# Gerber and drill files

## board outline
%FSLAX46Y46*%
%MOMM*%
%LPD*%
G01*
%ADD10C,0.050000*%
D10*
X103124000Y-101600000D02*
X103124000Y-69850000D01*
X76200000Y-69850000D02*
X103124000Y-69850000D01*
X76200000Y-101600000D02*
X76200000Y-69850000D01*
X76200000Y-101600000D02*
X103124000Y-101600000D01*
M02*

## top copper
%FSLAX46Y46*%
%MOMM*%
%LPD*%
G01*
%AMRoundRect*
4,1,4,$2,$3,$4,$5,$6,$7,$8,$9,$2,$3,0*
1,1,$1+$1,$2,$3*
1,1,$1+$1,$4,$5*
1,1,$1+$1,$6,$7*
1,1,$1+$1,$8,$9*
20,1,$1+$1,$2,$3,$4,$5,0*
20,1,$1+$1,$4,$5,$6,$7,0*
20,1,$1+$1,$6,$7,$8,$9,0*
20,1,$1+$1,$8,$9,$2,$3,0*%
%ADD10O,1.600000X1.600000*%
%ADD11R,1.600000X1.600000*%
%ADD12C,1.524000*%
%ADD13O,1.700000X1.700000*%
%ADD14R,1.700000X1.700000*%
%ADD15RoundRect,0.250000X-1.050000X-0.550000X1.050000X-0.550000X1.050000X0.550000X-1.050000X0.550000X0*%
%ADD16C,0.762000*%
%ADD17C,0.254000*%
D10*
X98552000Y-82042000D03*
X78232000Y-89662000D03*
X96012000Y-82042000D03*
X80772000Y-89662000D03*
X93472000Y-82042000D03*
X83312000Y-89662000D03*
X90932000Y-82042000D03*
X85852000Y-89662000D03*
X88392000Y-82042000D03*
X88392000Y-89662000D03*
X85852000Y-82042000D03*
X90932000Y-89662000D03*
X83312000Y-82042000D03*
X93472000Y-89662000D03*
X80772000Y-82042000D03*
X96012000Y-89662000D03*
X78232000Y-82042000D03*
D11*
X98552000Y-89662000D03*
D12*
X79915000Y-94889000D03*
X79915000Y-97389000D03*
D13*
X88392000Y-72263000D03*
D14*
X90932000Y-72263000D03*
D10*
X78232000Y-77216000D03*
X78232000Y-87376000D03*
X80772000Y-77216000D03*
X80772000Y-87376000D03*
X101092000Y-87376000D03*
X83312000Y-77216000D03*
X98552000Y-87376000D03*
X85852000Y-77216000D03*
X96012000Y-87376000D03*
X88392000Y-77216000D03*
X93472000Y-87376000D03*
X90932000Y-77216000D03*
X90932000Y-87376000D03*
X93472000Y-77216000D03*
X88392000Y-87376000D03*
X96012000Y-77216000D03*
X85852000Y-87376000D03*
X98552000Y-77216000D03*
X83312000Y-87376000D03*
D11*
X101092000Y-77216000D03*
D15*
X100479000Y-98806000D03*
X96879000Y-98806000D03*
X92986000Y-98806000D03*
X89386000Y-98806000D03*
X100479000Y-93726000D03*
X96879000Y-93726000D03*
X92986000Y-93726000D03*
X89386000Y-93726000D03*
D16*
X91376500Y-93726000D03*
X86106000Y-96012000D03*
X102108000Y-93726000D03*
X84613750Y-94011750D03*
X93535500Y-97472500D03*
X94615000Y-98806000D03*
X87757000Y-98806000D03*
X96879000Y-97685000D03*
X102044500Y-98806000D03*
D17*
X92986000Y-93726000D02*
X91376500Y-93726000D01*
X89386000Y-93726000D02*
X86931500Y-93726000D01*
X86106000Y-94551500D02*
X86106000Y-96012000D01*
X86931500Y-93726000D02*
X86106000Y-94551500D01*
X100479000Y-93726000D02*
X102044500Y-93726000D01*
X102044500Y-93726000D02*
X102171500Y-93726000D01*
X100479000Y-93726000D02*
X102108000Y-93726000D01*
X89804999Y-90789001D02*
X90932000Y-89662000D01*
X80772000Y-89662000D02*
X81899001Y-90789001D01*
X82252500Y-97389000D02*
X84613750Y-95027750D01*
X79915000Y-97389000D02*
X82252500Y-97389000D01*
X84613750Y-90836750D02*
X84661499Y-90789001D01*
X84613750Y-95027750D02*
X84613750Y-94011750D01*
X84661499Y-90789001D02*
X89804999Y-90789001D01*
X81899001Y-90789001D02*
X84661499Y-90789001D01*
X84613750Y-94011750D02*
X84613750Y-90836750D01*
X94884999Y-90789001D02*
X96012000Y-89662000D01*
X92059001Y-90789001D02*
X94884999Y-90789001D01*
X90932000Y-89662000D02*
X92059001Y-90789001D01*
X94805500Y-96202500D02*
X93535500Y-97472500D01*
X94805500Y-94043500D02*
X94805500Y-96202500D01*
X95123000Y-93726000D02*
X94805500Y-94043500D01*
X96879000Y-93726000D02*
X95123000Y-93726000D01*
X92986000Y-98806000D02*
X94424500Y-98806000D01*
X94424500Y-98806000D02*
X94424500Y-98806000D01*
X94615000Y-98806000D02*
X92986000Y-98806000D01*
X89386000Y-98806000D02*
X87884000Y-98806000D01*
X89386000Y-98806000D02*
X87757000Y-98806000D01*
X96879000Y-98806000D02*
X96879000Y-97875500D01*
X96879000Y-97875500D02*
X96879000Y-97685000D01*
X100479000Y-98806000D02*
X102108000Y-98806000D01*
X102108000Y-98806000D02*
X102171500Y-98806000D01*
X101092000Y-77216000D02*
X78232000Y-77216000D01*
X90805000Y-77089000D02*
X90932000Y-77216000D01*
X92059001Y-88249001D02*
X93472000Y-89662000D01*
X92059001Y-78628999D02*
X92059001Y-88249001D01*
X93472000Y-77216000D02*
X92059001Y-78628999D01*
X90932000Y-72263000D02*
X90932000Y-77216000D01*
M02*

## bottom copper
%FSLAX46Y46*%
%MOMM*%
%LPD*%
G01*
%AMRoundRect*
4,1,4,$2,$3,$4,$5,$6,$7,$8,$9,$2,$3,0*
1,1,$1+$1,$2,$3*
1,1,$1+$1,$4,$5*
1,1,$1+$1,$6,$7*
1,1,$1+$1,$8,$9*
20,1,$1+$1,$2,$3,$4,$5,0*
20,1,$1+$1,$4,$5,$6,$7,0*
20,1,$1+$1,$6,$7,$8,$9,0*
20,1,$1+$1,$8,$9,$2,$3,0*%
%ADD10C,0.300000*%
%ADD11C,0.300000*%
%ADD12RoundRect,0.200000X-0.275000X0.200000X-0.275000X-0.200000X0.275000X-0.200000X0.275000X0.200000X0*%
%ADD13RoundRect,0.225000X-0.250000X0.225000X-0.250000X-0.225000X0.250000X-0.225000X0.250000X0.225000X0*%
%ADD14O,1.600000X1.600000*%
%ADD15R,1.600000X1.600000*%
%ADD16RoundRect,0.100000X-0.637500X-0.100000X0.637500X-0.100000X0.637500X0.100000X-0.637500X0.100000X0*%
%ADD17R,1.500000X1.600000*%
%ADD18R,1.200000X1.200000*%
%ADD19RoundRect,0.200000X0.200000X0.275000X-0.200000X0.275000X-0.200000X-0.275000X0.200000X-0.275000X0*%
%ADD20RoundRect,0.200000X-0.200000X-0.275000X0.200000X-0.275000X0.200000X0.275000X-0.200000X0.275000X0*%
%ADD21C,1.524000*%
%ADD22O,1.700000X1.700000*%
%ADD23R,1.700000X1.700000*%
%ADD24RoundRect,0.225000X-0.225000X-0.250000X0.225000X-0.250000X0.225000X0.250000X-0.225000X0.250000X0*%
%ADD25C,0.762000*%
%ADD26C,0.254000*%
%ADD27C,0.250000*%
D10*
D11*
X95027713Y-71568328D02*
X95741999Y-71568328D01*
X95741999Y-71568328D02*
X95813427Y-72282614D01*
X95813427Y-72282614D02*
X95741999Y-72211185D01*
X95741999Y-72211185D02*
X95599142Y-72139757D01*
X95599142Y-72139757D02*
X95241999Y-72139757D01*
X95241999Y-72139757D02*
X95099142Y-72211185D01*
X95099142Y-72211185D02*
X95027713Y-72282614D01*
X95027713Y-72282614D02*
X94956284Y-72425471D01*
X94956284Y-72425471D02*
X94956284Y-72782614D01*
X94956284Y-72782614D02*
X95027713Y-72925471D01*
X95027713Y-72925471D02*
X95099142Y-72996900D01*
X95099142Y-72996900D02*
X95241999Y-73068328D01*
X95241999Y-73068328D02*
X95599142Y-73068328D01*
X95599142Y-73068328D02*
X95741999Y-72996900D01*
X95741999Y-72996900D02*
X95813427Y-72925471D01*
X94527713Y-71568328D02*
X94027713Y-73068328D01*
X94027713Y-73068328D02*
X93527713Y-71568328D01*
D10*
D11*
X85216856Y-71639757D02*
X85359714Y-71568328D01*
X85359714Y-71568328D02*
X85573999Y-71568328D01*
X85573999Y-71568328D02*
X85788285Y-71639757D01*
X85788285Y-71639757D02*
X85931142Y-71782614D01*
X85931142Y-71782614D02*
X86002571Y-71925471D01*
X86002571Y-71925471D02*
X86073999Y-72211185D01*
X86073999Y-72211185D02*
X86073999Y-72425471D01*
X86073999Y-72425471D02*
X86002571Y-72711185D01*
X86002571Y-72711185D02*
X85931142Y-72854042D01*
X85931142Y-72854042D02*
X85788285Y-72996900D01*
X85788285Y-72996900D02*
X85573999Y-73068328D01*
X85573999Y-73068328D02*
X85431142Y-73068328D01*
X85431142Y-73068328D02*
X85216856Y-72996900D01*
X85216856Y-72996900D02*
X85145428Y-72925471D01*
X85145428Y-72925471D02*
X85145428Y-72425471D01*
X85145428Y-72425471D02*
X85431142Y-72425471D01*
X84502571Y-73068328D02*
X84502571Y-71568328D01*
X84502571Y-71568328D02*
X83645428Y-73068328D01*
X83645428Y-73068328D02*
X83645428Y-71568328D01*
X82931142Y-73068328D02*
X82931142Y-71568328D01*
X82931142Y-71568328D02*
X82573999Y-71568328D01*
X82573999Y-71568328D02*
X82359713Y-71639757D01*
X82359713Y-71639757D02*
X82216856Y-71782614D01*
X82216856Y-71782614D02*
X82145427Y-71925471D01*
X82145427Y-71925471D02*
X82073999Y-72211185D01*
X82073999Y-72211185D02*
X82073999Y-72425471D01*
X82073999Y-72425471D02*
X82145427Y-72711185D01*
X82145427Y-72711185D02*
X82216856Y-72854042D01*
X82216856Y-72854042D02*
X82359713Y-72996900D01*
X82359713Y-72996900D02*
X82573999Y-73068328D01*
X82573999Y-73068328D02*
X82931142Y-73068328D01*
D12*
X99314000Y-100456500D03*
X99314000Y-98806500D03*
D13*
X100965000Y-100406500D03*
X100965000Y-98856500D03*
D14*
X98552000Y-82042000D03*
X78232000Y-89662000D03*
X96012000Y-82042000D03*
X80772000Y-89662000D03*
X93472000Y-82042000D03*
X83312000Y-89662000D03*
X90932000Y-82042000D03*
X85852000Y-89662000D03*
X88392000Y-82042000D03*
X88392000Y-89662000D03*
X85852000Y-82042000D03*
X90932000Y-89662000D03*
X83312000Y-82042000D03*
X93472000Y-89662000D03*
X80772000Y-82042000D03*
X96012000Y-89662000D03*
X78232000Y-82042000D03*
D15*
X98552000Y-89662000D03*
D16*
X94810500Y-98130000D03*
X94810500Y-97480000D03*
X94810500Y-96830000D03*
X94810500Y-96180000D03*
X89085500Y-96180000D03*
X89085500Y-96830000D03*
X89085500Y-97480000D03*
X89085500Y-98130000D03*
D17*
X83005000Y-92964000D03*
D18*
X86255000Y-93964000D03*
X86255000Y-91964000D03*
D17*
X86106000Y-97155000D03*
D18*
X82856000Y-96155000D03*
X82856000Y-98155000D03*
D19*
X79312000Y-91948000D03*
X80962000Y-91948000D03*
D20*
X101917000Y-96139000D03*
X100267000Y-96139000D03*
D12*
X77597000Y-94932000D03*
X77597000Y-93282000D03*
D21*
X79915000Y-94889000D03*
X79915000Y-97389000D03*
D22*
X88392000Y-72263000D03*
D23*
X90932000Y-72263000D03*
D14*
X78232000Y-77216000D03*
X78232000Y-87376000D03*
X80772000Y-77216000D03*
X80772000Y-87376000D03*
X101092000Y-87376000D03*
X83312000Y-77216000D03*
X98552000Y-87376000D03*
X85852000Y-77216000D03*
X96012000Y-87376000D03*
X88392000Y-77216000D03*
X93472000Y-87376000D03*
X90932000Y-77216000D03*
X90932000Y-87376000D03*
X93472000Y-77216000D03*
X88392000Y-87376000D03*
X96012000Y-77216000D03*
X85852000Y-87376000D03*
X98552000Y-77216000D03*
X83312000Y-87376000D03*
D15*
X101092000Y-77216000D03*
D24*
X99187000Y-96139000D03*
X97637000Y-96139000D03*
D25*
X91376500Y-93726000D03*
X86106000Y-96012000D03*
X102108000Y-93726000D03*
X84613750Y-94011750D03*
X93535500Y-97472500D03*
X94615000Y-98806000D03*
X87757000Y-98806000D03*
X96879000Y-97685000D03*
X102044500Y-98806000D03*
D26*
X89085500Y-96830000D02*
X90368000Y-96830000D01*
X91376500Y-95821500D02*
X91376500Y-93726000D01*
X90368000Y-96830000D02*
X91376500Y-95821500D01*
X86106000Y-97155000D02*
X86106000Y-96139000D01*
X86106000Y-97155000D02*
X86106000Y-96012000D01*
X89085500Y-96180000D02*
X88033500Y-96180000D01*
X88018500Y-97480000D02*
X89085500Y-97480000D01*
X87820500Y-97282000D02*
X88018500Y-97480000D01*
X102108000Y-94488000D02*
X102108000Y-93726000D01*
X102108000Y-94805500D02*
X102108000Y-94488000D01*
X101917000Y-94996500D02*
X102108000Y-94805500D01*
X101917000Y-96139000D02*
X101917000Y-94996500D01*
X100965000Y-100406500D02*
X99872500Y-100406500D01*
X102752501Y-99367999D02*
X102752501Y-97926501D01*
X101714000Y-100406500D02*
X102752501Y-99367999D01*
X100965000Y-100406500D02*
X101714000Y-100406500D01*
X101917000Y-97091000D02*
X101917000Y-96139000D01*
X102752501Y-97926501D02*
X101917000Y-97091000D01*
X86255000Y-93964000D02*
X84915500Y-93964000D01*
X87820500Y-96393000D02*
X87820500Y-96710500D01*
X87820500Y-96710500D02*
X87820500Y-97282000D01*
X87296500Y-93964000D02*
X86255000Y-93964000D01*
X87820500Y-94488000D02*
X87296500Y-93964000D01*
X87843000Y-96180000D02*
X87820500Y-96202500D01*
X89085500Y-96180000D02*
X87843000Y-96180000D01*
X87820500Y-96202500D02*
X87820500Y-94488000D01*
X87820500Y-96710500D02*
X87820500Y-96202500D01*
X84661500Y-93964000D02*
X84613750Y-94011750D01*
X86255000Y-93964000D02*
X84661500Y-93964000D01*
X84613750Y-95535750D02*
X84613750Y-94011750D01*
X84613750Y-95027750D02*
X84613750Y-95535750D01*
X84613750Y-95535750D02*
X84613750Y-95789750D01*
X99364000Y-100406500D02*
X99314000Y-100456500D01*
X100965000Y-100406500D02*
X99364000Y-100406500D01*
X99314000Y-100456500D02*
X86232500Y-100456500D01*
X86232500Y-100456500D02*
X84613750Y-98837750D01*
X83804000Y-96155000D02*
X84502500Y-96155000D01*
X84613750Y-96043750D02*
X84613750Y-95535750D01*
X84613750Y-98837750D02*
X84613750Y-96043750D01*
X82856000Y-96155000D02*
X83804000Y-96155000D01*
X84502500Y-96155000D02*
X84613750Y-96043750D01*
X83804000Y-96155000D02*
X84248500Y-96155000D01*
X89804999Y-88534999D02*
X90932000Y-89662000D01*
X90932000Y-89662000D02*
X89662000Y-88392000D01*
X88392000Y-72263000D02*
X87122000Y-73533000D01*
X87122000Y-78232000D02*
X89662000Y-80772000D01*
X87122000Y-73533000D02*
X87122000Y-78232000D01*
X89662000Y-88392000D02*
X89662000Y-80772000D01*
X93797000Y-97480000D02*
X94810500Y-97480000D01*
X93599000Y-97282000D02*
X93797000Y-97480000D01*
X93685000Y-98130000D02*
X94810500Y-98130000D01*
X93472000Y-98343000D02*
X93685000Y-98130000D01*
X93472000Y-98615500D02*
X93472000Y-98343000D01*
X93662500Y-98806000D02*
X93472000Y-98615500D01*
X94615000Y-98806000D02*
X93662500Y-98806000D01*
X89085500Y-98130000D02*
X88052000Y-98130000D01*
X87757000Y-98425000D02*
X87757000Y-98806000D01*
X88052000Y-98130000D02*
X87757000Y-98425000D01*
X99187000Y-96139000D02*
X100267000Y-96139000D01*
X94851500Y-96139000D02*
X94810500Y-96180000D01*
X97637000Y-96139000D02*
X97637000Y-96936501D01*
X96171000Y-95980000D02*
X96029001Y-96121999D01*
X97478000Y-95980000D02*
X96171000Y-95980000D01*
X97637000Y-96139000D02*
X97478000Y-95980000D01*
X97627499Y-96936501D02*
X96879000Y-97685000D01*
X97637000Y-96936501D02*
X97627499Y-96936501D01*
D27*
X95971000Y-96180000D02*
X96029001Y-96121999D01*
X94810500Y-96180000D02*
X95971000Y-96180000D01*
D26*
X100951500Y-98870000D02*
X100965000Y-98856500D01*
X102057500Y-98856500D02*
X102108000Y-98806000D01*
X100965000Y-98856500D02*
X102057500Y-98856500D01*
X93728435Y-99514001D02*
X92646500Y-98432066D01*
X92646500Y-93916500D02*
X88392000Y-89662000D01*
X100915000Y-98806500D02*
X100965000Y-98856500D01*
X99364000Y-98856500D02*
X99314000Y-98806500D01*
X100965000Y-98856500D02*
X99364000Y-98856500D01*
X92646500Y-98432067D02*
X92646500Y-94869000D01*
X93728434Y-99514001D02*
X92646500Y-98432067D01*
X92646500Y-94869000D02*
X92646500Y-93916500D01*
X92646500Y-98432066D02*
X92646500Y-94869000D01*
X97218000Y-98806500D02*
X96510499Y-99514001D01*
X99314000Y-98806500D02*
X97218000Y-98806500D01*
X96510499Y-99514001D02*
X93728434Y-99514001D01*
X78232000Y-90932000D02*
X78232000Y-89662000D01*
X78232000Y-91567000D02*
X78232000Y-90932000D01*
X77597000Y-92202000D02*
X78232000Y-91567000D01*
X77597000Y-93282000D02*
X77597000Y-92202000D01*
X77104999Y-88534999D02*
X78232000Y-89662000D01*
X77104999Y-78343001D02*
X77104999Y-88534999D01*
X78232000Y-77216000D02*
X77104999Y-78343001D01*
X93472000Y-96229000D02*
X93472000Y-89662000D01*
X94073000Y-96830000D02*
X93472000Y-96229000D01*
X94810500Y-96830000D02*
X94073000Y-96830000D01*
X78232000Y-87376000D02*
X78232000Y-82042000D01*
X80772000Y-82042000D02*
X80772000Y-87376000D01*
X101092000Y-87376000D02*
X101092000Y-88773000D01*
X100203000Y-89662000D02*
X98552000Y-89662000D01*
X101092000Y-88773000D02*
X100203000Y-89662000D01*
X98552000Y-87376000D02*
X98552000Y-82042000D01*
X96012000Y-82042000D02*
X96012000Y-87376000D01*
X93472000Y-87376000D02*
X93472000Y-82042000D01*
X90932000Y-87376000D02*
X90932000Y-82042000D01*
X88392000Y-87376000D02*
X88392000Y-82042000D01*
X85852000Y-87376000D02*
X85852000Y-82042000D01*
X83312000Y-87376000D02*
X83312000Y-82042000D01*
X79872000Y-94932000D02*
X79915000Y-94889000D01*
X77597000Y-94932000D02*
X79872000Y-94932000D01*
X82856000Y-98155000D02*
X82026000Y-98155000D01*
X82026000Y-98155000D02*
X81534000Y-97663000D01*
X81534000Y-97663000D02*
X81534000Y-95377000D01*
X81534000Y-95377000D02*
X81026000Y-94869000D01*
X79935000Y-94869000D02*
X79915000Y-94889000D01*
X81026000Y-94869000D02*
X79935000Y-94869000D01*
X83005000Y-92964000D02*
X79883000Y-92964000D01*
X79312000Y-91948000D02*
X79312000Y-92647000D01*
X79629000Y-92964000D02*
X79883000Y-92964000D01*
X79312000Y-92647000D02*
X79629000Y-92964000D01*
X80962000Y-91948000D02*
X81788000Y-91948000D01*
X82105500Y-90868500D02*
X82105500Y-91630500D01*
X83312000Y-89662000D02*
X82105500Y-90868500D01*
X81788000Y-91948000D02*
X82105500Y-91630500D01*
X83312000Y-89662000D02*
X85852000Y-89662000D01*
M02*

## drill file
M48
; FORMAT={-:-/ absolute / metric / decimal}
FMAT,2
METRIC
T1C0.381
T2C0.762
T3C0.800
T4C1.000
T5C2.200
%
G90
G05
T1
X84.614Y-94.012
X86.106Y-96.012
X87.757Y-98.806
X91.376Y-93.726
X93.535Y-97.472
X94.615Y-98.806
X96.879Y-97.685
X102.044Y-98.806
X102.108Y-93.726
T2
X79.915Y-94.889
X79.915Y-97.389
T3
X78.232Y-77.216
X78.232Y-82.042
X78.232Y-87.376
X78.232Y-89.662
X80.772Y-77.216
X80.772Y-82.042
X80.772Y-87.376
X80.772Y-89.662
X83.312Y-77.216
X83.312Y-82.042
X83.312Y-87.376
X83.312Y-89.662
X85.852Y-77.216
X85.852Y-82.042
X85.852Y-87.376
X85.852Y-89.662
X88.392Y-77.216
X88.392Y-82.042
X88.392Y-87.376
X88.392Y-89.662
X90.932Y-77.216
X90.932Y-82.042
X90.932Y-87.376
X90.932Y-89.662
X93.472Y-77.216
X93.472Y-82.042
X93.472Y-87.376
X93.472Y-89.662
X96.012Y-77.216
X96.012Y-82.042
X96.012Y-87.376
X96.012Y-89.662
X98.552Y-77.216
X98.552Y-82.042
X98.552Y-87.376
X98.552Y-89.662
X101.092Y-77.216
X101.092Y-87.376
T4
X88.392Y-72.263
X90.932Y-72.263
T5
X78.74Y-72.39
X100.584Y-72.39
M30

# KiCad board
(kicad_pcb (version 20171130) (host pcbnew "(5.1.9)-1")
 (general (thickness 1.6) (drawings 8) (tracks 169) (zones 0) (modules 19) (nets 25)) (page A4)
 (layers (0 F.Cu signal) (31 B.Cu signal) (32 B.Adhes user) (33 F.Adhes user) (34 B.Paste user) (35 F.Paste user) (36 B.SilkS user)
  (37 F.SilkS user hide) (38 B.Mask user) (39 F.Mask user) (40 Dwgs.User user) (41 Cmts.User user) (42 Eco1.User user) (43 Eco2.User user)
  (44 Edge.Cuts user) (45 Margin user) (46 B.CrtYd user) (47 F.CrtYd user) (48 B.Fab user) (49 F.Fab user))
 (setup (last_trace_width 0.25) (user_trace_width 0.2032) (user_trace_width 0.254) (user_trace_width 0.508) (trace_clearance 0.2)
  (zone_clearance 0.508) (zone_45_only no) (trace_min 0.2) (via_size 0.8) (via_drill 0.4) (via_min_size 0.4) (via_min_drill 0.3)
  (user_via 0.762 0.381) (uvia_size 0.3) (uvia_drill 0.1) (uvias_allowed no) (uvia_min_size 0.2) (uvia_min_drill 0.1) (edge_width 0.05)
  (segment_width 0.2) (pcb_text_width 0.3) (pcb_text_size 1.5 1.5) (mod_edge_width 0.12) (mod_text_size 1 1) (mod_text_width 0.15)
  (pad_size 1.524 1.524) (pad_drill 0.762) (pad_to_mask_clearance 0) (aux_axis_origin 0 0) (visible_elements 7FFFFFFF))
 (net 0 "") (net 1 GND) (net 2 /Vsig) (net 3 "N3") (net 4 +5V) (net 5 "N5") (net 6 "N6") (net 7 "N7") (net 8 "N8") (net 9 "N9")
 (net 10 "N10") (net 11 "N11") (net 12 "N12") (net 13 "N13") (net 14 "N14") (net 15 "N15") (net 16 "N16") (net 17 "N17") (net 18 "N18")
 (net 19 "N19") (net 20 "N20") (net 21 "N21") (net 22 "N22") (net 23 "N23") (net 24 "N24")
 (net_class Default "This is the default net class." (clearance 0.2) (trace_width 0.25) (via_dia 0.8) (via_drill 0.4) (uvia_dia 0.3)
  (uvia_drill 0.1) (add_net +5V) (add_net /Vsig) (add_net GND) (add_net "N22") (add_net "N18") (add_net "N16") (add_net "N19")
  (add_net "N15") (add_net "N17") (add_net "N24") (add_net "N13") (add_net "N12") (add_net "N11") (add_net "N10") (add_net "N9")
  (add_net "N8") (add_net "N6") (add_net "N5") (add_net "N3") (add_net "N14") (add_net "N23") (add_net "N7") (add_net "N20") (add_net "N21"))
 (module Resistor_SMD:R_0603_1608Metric (layer B.Cu) (at 99.314 99.6315 270)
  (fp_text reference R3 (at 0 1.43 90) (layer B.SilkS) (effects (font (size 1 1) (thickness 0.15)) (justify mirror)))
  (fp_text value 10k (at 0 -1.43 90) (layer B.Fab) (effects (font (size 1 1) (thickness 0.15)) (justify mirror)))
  (pad 2 smd roundrect (at 0.825 0 270) (size 0.8 0.95) (layers B.Cu B.Paste B.Mask) (roundrect_rratio 0.25) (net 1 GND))
  (pad 1 smd roundrect (at -0.825 0 270) (size 0.8 0.95) (layers B.Cu B.Paste B.Mask) (roundrect_rratio 0.25) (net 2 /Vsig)))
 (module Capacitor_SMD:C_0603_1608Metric (layer B.Cu) (at 100.965 99.6315 270)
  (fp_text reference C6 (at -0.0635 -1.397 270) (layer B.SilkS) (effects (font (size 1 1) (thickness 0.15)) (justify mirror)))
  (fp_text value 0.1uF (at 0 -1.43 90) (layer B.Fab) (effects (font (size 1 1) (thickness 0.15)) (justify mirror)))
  (pad 2 smd roundrect (at 0.775 0 270) (size 0.9 0.95) (layers B.Cu B.Paste B.Mask) (roundrect_rratio 0.25) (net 1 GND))
  (pad 1 smd roundrect (at -0.775 0 270) (size 0.9 0.95) (layers B.Cu B.Paste B.Mask) (roundrect_rratio 0.25) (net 2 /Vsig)))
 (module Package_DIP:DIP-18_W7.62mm (layer B.Cu) (at 98.552 89.662 90)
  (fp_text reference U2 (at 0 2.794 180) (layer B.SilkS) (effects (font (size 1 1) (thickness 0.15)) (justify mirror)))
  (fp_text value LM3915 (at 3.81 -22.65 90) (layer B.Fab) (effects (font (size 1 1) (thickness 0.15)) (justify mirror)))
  (pad 18 thru_hole oval (at 7.62 0 90) (size 1.6 1.6) (drill 0.8) (layers *.Cu *.Mask) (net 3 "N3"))
  (pad 9 thru_hole oval (at 0 -20.32 90) (size 1.6 1.6) (drill 0.8) (layers *.Cu *.Mask) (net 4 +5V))
  (pad 17 thru_hole oval (at 7.62 -2.54 90) (size 1.6 1.6) (drill 0.8) (layers *.Cu *.Mask) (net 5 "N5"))
  (pad 8 thru_hole oval (at 0 -17.78 90) (size 1.6 1.6) (drill 0.8) (layers *.Cu *.Mask) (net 1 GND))
  (pad 16 thru_hole oval (at 7.62 -5.08 90) (size 1.6 1.6) (drill 0.8) (layers *.Cu *.Mask) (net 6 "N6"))
  (pad 7 thru_hole oval (at 0 -15.24 90) (size 1.6 1.6) (drill 0.8) (layers *.Cu *.Mask) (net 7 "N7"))
  (pad 15 thru_hole oval (at 7.62 -7.62 90) (size 1.6 1.6) (drill 0.8) (layers *.Cu *.Mask) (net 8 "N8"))
  (pad 6 thru_hole oval (at 0 -12.7 90) (size 1.6 1.6) (drill 0.8) (layers *.Cu *.Mask) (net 7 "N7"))
  (pad 14 thru_hole oval (at 7.62 -10.16 90) (size 1.6 1.6) (drill 0.8) (layers *.Cu *.Mask) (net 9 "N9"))
  (pad 5 thru_hole oval (at 0 -10.16 90) (size 1.6 1.6) (drill 0.8) (layers *.Cu *.Mask) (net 2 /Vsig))
  (pad 13 thru_hole oval (at 7.62 -12.7 90) (size 1.6 1.6) (drill 0.8) (layers *.Cu *.Mask) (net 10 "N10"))
  (pad 4 thru_hole oval (at 0 -7.62 90) (size 1.6 1.6) (drill 0.8) (layers *.Cu *.Mask) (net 1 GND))
  (pad 12 thru_hole oval (at 7.62 -15.24 90) (size 1.6 1.6) (drill 0.8) (layers *.Cu *.Mask) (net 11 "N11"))
  (pad 3 thru_hole oval (at 0 -5.08 90) (size 1.6 1.6) (drill 0.8) (layers *.Cu *.Mask) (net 4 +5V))
  (pad 11 thru_hole oval (at 7.62 -17.78 90) (size 1.6 1.6) (drill 0.8) (layers *.Cu *.Mask) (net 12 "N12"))
  (pad 2 thru_hole oval (at 0 -2.54 90) (size 1.6 1.6) (drill 0.8) (layers *.Cu *.Mask) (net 1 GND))
  (pad 10 thru_hole oval (at 7.62 -20.32 90) (size 1.6 1.6) (drill 0.8) (layers *.Cu *.Mask) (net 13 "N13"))
  (pad 1 thru_hole rect (at 0 0 90) (size 1.6 1.6) (drill 0.8) (layers *.Cu *.Mask) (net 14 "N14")))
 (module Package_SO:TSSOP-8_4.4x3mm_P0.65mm (layer B.Cu) (at 91.948 97.155)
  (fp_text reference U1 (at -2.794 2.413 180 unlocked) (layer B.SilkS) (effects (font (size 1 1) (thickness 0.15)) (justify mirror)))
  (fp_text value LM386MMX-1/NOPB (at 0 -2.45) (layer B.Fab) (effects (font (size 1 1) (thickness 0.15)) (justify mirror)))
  (pad 8 smd roundrect (at 2.8625 0.975) (size 1.475 0.4) (layers B.Cu B.Paste B.Mask) (roundrect_rratio 0.25) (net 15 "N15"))
  (pad 7 smd roundrect (at 2.8625 0.325) (size 1.475 0.4) (layers B.Cu B.Paste B.Mask) (roundrect_rratio 0.25) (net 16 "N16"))
  (pad 6 smd roundrect (at 2.8625 -0.325) (size 1.475 0.4) (layers B.Cu B.Paste B.Mask) (roundrect_rratio 0.25) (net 4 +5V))
  (pad 5 smd roundrect (at 2.8625 -0.975) (size 1.475 0.4) (layers B.Cu B.Paste B.Mask) (roundrect_rratio 0.25) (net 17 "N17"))
  (pad 4 smd roundrect (at -2.8625 -0.975) (size 1.475 0.4) (layers B.Cu B.Paste B.Mask) (roundrect_rratio 0.25) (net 1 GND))
  (pad 3 smd roundrect (at -2.8625 -0.325) (size 1.475 0.4) (layers B.Cu B.Paste B.Mask) (roundrect_rratio 0.25) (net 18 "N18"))
  (pad 2 smd roundrect (at -2.8625 0.325) (size 1.475 0.4) (layers B.Cu B.Paste B.Mask) (roundrect_rratio 0.25) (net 1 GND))
  (pad 1 smd roundrect (at -2.8625 0.975) (size 1.475 0.4) (layers B.Cu B.Paste B.Mask) (roundrect_rratio 0.25) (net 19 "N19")))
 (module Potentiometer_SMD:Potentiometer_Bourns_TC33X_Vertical (layer B.Cu) (at 84.455 92.964 180)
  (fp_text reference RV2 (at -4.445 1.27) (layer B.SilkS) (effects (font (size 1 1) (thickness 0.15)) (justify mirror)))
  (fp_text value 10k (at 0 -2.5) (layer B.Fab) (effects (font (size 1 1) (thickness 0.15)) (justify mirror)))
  (pad 2 smd rect (at 1.45 0 180) (size 1.5 1.6) (layers B.Cu B.Paste B.Mask) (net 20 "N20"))
  (pad 3 smd rect (at -1.8 -1 180) (size 1.2 1.2) (layers B.Cu B.Paste B.Mask) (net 1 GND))
  (pad 1 smd rect (at -1.8 1 180) (size 1.2 1.2) (layers B.Cu B.Paste B.Mask) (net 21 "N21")))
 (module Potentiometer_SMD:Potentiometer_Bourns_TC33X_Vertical (layer B.Cu) (at 84.656 97.155)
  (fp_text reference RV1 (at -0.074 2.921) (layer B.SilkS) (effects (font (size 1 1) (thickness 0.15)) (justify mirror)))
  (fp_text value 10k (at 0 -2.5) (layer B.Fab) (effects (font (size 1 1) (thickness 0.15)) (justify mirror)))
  (pad 2 smd rect (at 1.45 0) (size 1.5 1.6) (layers B.Cu B.Paste B.Mask) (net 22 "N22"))
  (pad 3 smd rect (at -1.8 -1) (size 1.2 1.2) (layers B.Cu B.Paste B.Mask) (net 1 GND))
  (pad 1 smd rect (at -1.8 1) (size 1.2 1.2) (layers B.Cu B.Paste B.Mask) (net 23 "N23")))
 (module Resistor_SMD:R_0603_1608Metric (layer B.Cu) (at 80.137 91.948 180)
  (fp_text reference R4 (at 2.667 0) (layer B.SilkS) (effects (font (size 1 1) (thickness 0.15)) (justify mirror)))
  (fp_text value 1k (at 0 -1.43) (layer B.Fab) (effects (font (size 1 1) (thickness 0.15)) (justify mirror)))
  (pad 2 smd roundrect (at 0.825 0 180) (size 0.8 0.95) (layers B.Cu B.Paste B.Mask) (roundrect_rratio 0.25) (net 20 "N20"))
  (pad 1 smd roundrect (at -0.825 0 180) (size 0.8 0.95) (layers B.Cu B.Paste B.Mask) (roundrect_rratio 0.25) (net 7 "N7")))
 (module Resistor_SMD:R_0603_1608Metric (layer B.Cu) (at 101.092 96.139)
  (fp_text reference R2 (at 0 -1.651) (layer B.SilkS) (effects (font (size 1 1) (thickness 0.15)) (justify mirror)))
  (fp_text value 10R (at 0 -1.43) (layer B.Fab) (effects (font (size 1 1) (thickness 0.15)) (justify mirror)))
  (pad 2 smd roundrect (at 0.825 0) (size 0.8 0.95) (layers B.Cu B.Paste B.Mask) (roundrect_rratio 0.25) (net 1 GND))
  (pad 1 smd roundrect (at -0.825 0) (size 0.8 0.95) (layers B.Cu B.Paste B.Mask) (roundrect_rratio 0.25) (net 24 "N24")))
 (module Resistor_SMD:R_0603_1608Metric (layer B.Cu) (at 77.597 94.107 270)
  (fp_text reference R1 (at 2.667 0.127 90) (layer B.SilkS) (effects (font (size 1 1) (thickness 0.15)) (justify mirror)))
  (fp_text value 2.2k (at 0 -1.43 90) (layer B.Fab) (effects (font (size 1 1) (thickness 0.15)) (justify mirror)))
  (pad 2 smd roundrect (at 0.825 0 270) (size 0.8 0.95) (layers B.Cu B.Paste B.Mask) (roundrect_rratio 0.25) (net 23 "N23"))
  (pad 1 smd roundrect (at -0.825 0 270) (size 0.8 0.95) (layers B.Cu B.Paste B.Mask) (roundrect_rratio 0.25) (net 4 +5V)))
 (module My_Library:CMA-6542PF (layer F.Cu) (at 81.915 96.139 180)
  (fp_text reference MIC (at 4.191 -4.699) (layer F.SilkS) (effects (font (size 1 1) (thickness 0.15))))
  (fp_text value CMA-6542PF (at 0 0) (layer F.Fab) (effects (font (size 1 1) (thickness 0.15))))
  (pad 2 thru_hole circle (at 2 1.25 180) (size 1.524 1.524) (drill 0.762) (layers *.Cu *.Mask) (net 23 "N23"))
  (pad 1 thru_hole circle (at 2 -1.25 270) (size 1.524 1.524) (drill 0.762) (layers *.Cu *.Mask) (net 1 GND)))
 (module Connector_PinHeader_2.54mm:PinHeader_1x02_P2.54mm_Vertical (layer B.Cu) (at 90.932 72.263 90)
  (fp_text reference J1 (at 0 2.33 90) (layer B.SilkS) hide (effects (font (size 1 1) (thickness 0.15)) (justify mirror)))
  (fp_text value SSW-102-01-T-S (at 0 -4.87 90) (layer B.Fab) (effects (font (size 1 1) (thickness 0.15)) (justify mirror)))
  (pad 2 thru_hole oval (at 0 -2.54 90) (size 1.7 1.7) (drill 1) (layers *.Cu *.Mask) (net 1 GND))
  (pad 1 thru_hole rect (at 0 0 90) (size 1.7 1.7) (drill 1) (layers *.Cu *.Mask) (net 4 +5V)))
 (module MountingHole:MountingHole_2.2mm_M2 (layer F.Cu) (at 100.584 72.39)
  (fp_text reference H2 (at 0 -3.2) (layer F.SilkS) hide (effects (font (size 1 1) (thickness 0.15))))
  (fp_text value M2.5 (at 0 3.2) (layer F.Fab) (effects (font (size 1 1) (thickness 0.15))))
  (pad 1 np_thru_hole circle (at 0 0) (size 2.2 2.2) (drill 2.2) (layers *.Cu *.Mask)))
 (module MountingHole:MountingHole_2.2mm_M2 (layer F.Cu) (at 78.74 72.39)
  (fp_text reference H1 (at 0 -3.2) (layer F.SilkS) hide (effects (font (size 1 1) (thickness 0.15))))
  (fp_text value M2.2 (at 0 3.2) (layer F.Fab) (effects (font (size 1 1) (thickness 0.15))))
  (pad 1 np_thru_hole circle (at 0 0) (size 2.2 2.2) (drill 2.2) (layers *.Cu *.Mask)))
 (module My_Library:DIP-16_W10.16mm (layer F.Cu) (at 101.092 77.216 270)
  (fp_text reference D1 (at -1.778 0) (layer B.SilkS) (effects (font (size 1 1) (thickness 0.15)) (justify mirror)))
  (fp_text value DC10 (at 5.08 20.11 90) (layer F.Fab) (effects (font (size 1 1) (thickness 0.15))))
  (pad 10 thru_hole oval (at 0 22.86 270) (size 1.6 1.6) (drill 0.8) (layers *.Cu *.Mask) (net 4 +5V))
  (pad 11 thru_hole oval (at 10.16 22.86 270) (size 1.6 1.6) (drill 0.8) (layers *.Cu *.Mask) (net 13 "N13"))
  (pad 9 thru_hole oval (at 0 20.32 270) (size 1.6 1.6) (drill 0.8) (layers *.Cu *.Mask) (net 4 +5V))
  (pad 12 thru_hole oval (at 10.16 20.32 270) (size 1.6 1.6) (drill 0.8) (layers *.Cu *.Mask) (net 12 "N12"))
  (pad 20 thru_hole oval (at 10.16 0 270) (size 1.6 1.6) (drill 0.8) (layers *.Cu *.Mask) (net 14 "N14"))
  (pad 8 thru_hole oval (at 0 17.78 270) (size 1.6 1.6) (drill 0.8) (layers *.Cu *.Mask) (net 4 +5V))
  (pad 19 thru_hole oval (at 10.16 2.54 270) (size 1.6 1.6) (drill 0.8) (layers *.Cu *.Mask) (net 3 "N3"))
  (pad 7 thru_hole oval (at 0 15.24 270) (size 1.6 1.6) (drill 0.8) (layers *.Cu *.Mask) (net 4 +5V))
  (pad 18 thru_hole oval (at 10.16 5.08 270) (size 1.6 1.6) (drill 0.8) (layers *.Cu *.Mask) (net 5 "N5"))
  (pad 6 thru_hole oval (at 0 12.7 270) (size 1.6 1.6) (drill 0.8) (layers *.Cu *.Mask) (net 4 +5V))
  (pad 17 thru_hole oval (at 10.16 7.62 270) (size 1.6 1.6) (drill 0.8) (layers *.Cu *.Mask) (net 6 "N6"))
  (pad 5 thru_hole oval (at 0 10.16 270) (size 1.6 1.6) (drill 0.8) (layers *.Cu *.Mask) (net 4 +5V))
  (pad 16 thru_hole oval (at 10.16 10.16 270) (size 1.6 1.6) (drill 0.8) (layers *.Cu *.Mask) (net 8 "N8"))
  (pad 4 thru_hole oval (at 0 7.62 270) (size 1.6 1.6) (drill 0.8) (layers *.Cu *.Mask) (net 4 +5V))
  (pad 15 thru_hole oval (at 10.16 12.7 270) (size 1.6 1.6) (drill 0.8) (layers *.Cu *.Mask) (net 9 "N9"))
  (pad 3 thru_hole oval (at 0 5.08 270) (size 1.6 1.6) (drill 0.8) (layers *.Cu *.Mask) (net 4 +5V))
  (pad 14 thru_hole oval (at 10.16 15.24 270) (size 1.6 1.6) (drill 0.8) (layers *.Cu *.Mask) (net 10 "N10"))
  (pad 2 thru_hole oval (at 0 2.54 270) (size 1.6 1.6) (drill 0.8) (layers *.Cu *.Mask) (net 4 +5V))
  (pad 13 thru_hole oval (at 10.16 17.78 270) (size 1.6 1.6) (drill 0.8) (layers *.Cu *.Mask) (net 11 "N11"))
  (pad 1 thru_hole rect (at 0 0 270) (size 1.6 1.6) (drill 0.8) (layers *.Cu *.Mask) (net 4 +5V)))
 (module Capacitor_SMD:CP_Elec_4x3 (layer F.Cu) (at 98.679 98.806)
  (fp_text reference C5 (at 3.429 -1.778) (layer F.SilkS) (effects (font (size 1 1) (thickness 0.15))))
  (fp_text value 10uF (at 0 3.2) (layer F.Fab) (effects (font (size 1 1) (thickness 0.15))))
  (pad 2 smd roundrect (at 1.8 0) (size 2.6 1.6) (layers F.Cu F.Paste F.Mask) (roundrect_rratio 0.15625) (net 2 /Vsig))
  (pad 1 smd roundrect (at -1.8 0) (size 2.6 1.6) (layers F.Cu F.Paste F.Mask) (roundrect_rratio 0.15625) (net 17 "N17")))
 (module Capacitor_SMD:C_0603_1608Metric (layer B.Cu) (at 98.412 96.139)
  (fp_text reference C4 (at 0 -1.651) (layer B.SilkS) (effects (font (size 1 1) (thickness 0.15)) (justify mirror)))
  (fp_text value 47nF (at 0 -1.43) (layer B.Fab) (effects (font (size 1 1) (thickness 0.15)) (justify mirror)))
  (pad 2 smd roundrect (at 0.775 0) (size 0.9 0.95) (layers B.Cu B.Paste B.Mask) (roundrect_rratio 0.25) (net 24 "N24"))
  (pad 1 smd roundrect (at -0.775 0) (size 0.9 0.95) (layers B.Cu B.Paste B.Mask) (roundrect_rratio 0.25) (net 17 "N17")))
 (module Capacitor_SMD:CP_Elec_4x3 (layer F.Cu) (at 91.186 98.806)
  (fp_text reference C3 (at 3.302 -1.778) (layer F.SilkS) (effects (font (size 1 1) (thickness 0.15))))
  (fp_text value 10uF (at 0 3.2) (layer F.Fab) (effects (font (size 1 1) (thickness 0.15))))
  (pad 2 smd roundrect (at 1.8 0) (size 2.6 1.6) (layers F.Cu F.Paste F.Mask) (roundrect_rratio 0.15625) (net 15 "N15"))
  (pad 1 smd roundrect (at -1.8 0) (size 2.6 1.6) (layers F.Cu F.Paste F.Mask) (roundrect_rratio 0.15625) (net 19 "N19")))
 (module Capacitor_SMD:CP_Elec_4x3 (layer F.Cu) (at 98.679 93.726)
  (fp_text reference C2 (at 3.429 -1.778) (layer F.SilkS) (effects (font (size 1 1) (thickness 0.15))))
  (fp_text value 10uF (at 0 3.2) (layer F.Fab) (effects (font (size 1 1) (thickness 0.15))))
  (pad 2 smd roundrect (at 1.8 0) (size 2.6 1.6) (layers F.Cu F.Paste F.Mask) (roundrect_rratio 0.15625) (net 1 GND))
  (pad 1 smd roundrect (at -1.8 0) (size 2.6 1.6) (layers F.Cu F.Paste F.Mask) (roundrect_rratio 0.15625) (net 16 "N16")))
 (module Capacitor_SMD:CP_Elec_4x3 (layer F.Cu) (at 91.186 93.726)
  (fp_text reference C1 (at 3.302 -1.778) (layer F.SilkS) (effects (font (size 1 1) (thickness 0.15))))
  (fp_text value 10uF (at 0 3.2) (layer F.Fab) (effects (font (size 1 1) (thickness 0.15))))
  (pad 2 smd roundrect (at 1.8 0) (size 2.6 1.6) (layers F.Cu F.Paste F.Mask) (roundrect_rratio 0.15625) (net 18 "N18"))
  (pad 1 smd roundrect (at -1.8 0) (size 2.6 1.6) (layers F.Cu F.Paste F.Mask) (roundrect_rratio 0.15625) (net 22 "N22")))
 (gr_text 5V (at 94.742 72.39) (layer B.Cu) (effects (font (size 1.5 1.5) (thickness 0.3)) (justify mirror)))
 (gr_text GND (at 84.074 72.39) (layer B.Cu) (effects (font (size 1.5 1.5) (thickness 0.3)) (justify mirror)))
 (gr_line (start 103.124 101.6) (end 103.124 69.85) (layer Edge.Cuts) (width 0.05))
 (gr_line (start 76.2 69.85) (end 103.124 69.85) (layer Edge.Cuts) (width 0.05))
 (gr_line (start 76.2 101.6) (end 76.2 69.85) (layer Edge.Cuts) (width 0.05))
 (gr_line (start 76.2 101.6) (end 103.124 101.6) (layer Edge.Cuts) (width 0.05))
 (via (at 91.3765 93.726) (size 0.762) (drill 0.381) (layers F.Cu B.Cu) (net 18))
 (segment (start 92.986 93.726) (end 91.3765 93.726) (width 0.254) (layer F.Cu) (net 18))
 (segment (start 89.0855 96.83) (end 90.368 96.83) (width 0.254) (layer B.Cu) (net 18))
 (segment (start 91.3765 95.8215) (end 91.3765 93.726) (width 0.254) (layer B.Cu) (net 18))
 (segment (start 90.368 96.83) (end 91.3765 95.8215) (width 0.254) (layer B.Cu) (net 18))
 (via (at 86.106 96.012) (size 0.762) (drill 0.381) (layers F.Cu B.Cu) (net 22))
 (segment (start 86.106 97.155) (end 86.106 96.139) (width 0.254) (layer B.Cu) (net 22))
 (segment (start 86.106 97.155) (end 86.106 96.012) (width 0.254) (layer B.Cu) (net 22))
 (segment (start 89.386 93.726) (end 86.9315 93.726) (width 0.254) (layer F.Cu) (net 22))
 (segment (start 86.106 94.5515) (end 86.106 96.012) (width 0.254) (layer F.Cu) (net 22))
 (segment (start 86.9315 93.726) (end 86.106 94.5515) (width 0.254) (layer F.Cu) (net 22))
 (segment (start 89.0855 96.18) (end 88.0335 96.18) (width 0.254) (layer B.Cu) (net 1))
 (segment (start 88.0185 97.48) (end 89.0855 97.48) (width 0.254) (layer B.Cu) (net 1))
 (segment (start 87.8205 97.282) (end 88.0185 97.48) (width 0.254) (layer B.Cu) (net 1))
 (segment (start 100.479 93.726) (end 102.0445 93.726) (width 0.254) (layer F.Cu) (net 1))
 (segment (start 102.0445 93.726) (end 102.1715 93.726) (width 0.254) (layer F.Cu) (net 1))
 (via (at 102.108 93.726) (size 0.762) (drill 0.381) (layers F.Cu B.Cu) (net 1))
 (segment (start 102.108 94.488) (end 102.108 93.726) (width 0.254) (layer B.Cu) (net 1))
 (segment (start 102.108 94.8055) (end 102.108 94.488) (width 0.254) (layer B.Cu) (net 1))
 (segment (start 101.917 94.9965) (end 102.108 94.8055) (width 0.254) (layer B.Cu) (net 1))
 (segment (start 101.917 96.139) (end 101.917 94.9965) (width 0.254) (layer B.Cu) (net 1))
 (segment (start 100.479 93.726) (end 102.108 93.726) (width 0.254) (layer F.Cu) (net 1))
 (segment (start 100.965 100.4065) (end 99.8725 100.4065) (width 0.254) (layer B.Cu) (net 1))
 (segment (start 102.752501 99.367999) (end 102.752501 97.926501) (width 0.254) (layer B.Cu) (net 1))
 (segment (start 101.714 100.4065) (end 102.752501 99.367999) (width 0.254) (layer B.Cu) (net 1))
 (segment (start 100.965 100.4065) (end 101.714 100.4065) (width 0.254) (layer B.Cu) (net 1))
 (segment (start 101.917 97.091) (end 101.917 96.139) (width 0.254) (layer B.Cu) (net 1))
 (segment (start 102.752501 97.926501) (end 101.917 97.091) (width 0.254) (layer B.Cu) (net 1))
 (segment (start 89.804999 90.789001) (end 90.932 89.662) (width 0.254) (layer F.Cu) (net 1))
 (segment (start 80.772 89.662) (end 81.899001 90.789001) (width 0.254) (layer F.Cu) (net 1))
 (segment (start 86.255 93.964) (end 84.9155 93.964) (width 0.254) (layer B.Cu) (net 1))
 (segment (start 82.2525 97.389) (end 84.61375 95.02775) (width 0.254) (layer F.Cu) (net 1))
 (segment (start 79.915 97.389) (end 82.2525 97.389) (width 0.254) (layer F.Cu) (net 1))
 (segment (start 84.61375 90.83675) (end 84.661499 90.789001) (width 0.254) (layer F.Cu) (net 1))
 (segment (start 84.61375 95.02775) (end 84.61375 94.01175) (width 0.254) (layer F.Cu) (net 1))
 (segment (start 84.661499 90.789001) (end 89.804999 90.789001) (width 0.254) (layer F.Cu) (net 1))
 (segment (start 81.899001 90.789001) (end 84.661499 90.789001) (width 0.254) (layer F.Cu) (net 1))
 (segment (start 87.8205 96.393) (end 87.8205 96.7105) (width 0.254) (layer B.Cu) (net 1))
 (segment (start 87.8205 96.7105) (end 87.8205 97.282) (width 0.254) (layer B.Cu) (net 1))
 (segment (start 87.2965 93.964) (end 86.255 93.964) (width 0.254) (layer B.Cu) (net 1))
 (segment (start 87.8205 94.488) (end 87.2965 93.964) (width 0.254) (layer B.Cu) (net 1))
 (segment (start 87.843 96.18) (end 87.8205 96.2025) (width 0.254) (layer B.Cu) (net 1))
 (segment (start 89.0855 96.18) (end 87.843 96.18) (width 0.254) (layer B.Cu) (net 1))
 (segment (start 87.8205 96.2025) (end 87.8205 94.488) (width 0.254) (layer B.Cu) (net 1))
 (segment (start 87.8205 96.7105) (end 87.8205 96.2025) (width 0.254) (layer B.Cu) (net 1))
 (segment (start 84.61375 94.01175) (end 84.61375 90.83675) (width 0.254) (layer F.Cu) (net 1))
 (via (at 84.61375 94.01175) (size 0.762) (drill 0.381) (layers F.Cu B.Cu) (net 1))
 (segment (start 84.6615 93.964) (end 84.61375 94.01175) (width 0.254) (layer B.Cu) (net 1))
 (segment (start 86.255 93.964) (end 84.6615 93.964) (width 0.254) (layer B.Cu) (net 1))
 (segment (start 84.61375 95.53575) (end 84.61375 94.01175) (width 0.254) (layer B.Cu) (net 1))
 (segment (start 84.61375 95.02775) (end 84.61375 95.53575) (width 0.254) (layer B.Cu) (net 1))
 (segment (start 84.61375 95.53575) (end 84.61375 95.78975) (width 0.254) (layer B.Cu) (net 1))
 (segment (start 99.364 100.4065) (end 99.314 100.4565) (width 0.254) (layer B.Cu) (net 1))
 (segment (start 100.965 100.4065) (end 99.364 100.4065) (width 0.254) (layer B.Cu) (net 1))
 (segment (start 94.884999 90.789001) (end 96.012 89.662) (width 0.254) (layer F.Cu) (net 1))
 (segment (start 92.059001 90.789001) (end 94.884999 90.789001) (width 0.254) (layer F.Cu) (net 1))
 (segment (start 90.932 89.662) (end 92.059001 90.789001) (width 0.254) (layer F.Cu) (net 1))
 (segment (start 99.314 100.4565) (end 86.2325 100.4565) (width 0.254) (layer B.Cu) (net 1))
 (segment (start 86.2325 100.4565) (end 84.61375 98.83775) (width 0.254) (layer B.Cu) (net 1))
 (segment (start 83.804 96.155) (end 84.5025 96.155) (width 0.254) (layer B.Cu) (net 1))
 (segment (start 84.61375 96.04375) (end 84.61375 95.53575) (width 0.254) (layer B.Cu) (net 1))
 (segment (start 84.61375 98.83775) (end 84.61375 96.04375) (width 0.254) (layer B.Cu) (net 1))
 (segment (start 82.856 96.155) (end 83.804 96.155) (width 0.254) (layer B.Cu) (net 1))
 (segment (start 84.5025 96.155) (end 84.61375 96.04375) (width 0.254) (layer B.Cu) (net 1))
 (segment (start 83.804 96.155) (end 84.2485 96.155) (width 0.254) (layer B.Cu) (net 1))
 (segment (start 89.804999 88.534999) (end 90.932 89.662) (width 0.254) (layer B.Cu) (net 1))
 (segment (start 90.932 89.662) (end 89.662 88.392) (width 0.254) (layer B.Cu) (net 1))
 (segment (start 88.392 72.263) (end 87.122 73.533) (width 0.254) (layer B.Cu) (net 1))
 (segment (start 87.122 78.232) (end 89.662 80.772) (width 0.254) (layer B.Cu) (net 1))
 (segment (start 87.122 73.533) (end 87.122 78.232) (width 0.254) (layer B.Cu) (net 1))
 (segment (start 89.662 88.392) (end 89.662 80.772) (width 0.254) (layer B.Cu) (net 1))
 (segment (start 93.797 97.48) (end 94.8105 97.48) (width 0.254) (layer B.Cu) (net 16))
 (segment (start 93.599 97.282) (end 93.797 97.48) (width 0.254) (layer B.Cu) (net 16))
 (via (at 93.5355 97.4725) (size 0.762) (drill 0.381) (layers F.Cu B.Cu) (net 16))
 (segment (start 94.8055 96.2025) (end 93.5355 97.4725) (width 0.254) (layer F.Cu) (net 16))
 (segment (start 94.8055 94.0435) (end 94.8055 96.2025) (width 0.254) (layer F.Cu) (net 16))
 (segment (start 95.123 93.726) (end 94.8055 94.0435) (width 0.254) (layer F.Cu) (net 16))
 (segment (start 96.879 93.726) (end 95.123 93.726) (width 0.254) (layer F.Cu) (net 16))
 (segment (start 92.986 98.806) (end 94.4245 98.806) (width 0.254) (layer F.Cu) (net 15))
 (segment (start 94.4245 98.806) (end 94.4245 98.806) (width 0.254) (layer F.Cu) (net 15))
 (via (at 94.615 98.806) (size 0.762) (drill 0.381) (layers F.Cu B.Cu) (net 15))
 (segment (start 94.615 98.806) (end 92.986 98.806) (width 0.254) (layer F.Cu) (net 15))
 (segment (start 93.685 98.13) (end 94.8105 98.13) (width 0.254) (layer B.Cu) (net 15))
 (segment (start 93.472 98.343) (end 93.685 98.13) (width 0.254) (layer B.Cu) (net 15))
 (segment (start 93.472 98.6155) (end 93.472 98.343) (width 0.254) (layer B.Cu) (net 15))
 (segment (start 93.6625 98.806) (end 93.472 98.6155) (width 0.254) (layer B.Cu) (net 15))
 (segment (start 94.615 98.806) (end 93.6625 98.806) (width 0.254) (layer B.Cu) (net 15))
 (via (at 87.757 98.806) (size 0.762) (drill 0.381) (layers F.Cu B.Cu) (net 19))
 (segment (start 89.386 98.806) (end 87.884 98.806) (width 0.254) (layer F.Cu) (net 19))
 (segment (start 89.386 98.806) (end 87.757 98.806) (width 0.254) (layer F.Cu) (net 19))
 (segment (start 89.0855 98.13) (end 88.052 98.13) (width 0.254) (layer B.Cu) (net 19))
 (segment (start 87.757 98.425) (end 87.757 98.806) (width 0.254) (layer B.Cu) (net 19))
 (segment (start 88.052 98.13) (end 87.757 98.425) (width 0.254) (layer B.Cu) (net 19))
 (segment (start 99.187 96.139) (end 100.267 96.139) (width 0.254) (layer B.Cu) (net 24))
 (segment (start 94.8515 96.139) (end 94.8105 96.18) (width 0.254) (layer B.Cu) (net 17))
 (segment (start 97.637 96.139) (end 97.637 96.936501) (width 0.254) (layer B.Cu) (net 17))
 (segment (start 96.171 95.98) (end 96.029001 96.121999) (width 0.254) (layer B.Cu) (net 17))
 (segment (start 97.478 95.98) (end 96.171 95.98) (width 0.254) (layer B.Cu) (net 17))
 (segment (start 97.637 96.139) (end 97.478 95.98) (width 0.254) (layer B.Cu) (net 17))
 (segment (start 96.879 98.806) (end 96.879 97.8755) (width 0.254) (layer F.Cu) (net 17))
 (segment (start 96.879 97.8755) (end 96.879 97.685) (width 0.254) (layer F.Cu) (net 17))
 (via (at 96.879 97.685) (size 0.762) (drill 0.381) (layers F.Cu B.Cu) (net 17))
 (segment (start 97.627499 96.936501) (end 96.879 97.685) (width 0.254) (layer B.Cu) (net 17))
 (segment (start 97.637 96.936501) (end 97.627499 96.936501) (width 0.254) (layer B.Cu) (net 17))
 (segment (start 95.971 96.18) (end 96.029001 96.121999) (width 0.25) (layer B.Cu) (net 17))
 (segment (start 94.8105 96.18) (end 95.971 96.18) (width 0.25) (layer B.Cu) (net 17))
 (segment (start 100.9515 98.87) (end 100.965 98.8565) (width 0.254) (layer B.Cu) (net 2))
 (segment (start 100.479 98.806) (end 102.108 98.806) (width 0.254) (layer F.Cu) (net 2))
 (segment (start 102.108 98.806) (end 102.1715 98.806) (width 0.254) (layer F.Cu) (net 2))
 (via (at 102.0445 98.806) (size 0.762) (drill 0.381) (layers F.Cu B.Cu) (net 2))
 (segment (start 102.0575 98.8565) (end 102.108 98.806) (width 0.254) (layer B.Cu) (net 2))
 (segment (start 100.965 98.8565) (end 102.0575 98.8565) (width 0.254) (layer B.Cu) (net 2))
 (segment (start 93.728435 99.514001) (end 92.6465 98.432066) (width 0.254) (layer B.Cu) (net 2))
 (segment (start 92.6465 93.9165) (end 88.392 89.662) (width 0.254) (layer B.Cu) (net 2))
 (segment (start 100.915 98.8065) (end 100.965 98.8565) (width 0.254) (layer B.Cu) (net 2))
 (segment (start 99.364 98.8565) (end 99.314 98.8065) (width 0.254) (layer B.Cu) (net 2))
 (segment (start 100.965 98.8565) (end 99.364 98.8565) (width 0.254) (layer B.Cu) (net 2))
 (segment (start 92.6465 98.432067) (end 92.6465 94.869) (width 0.254) (layer B.Cu) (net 2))
 (segment (start 93.728434 99.514001) (end 92.6465 98.432067) (width 0.254) (layer B.Cu) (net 2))
 (segment (start 92.6465 94.869) (end 92.6465 93.9165) (width 0.254) (layer B.Cu) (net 2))
 (segment (start 92.6465 98.432066) (end 92.6465 94.869) (width 0.254) (layer B.Cu) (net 2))
 (segment (start 97.218 98.8065) (end 96.510499 99.514001) (width 0.254) (layer B.Cu) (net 2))
 (segment (start 99.314 98.8065) (end 97.218 98.8065) (width 0.254) (layer B.Cu) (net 2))
 (segment (start 96.510499 99.514001) (end 93.728434 99.514001) (width 0.254) (layer B.Cu) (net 2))
 (segment (start 78.232 90.932) (end 78.232 89.662) (width 0.254) (layer B.Cu) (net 4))
 (segment (start 78.232 91.567) (end 78.232 90.932) (width 0.254) (layer B.Cu) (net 4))
 (segment (start 77.597 92.202) (end 78.232 91.567) (width 0.254) (layer B.Cu) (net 4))
 (segment (start 77.597 93.282) (end 77.597 92.202) (width 0.254) (layer B.Cu) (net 4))
 (segment (start 101.092 77.216) (end 78.232 77.216) (width 0.254) (layer F.Cu) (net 4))
 (segment (start 90.805 77.089) (end 90.932 77.216) (width 0.254) (layer F.Cu) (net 4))
 (segment (start 92.059001 88.249001) (end 93.472 89.662) (width 0.254) (layer F.Cu) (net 4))
 (segment (start 92.059001 78.628999) (end 92.059001 88.249001) (width 0.254) (layer F.Cu) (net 4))
 (segment (start 93.472 77.216) (end 92.059001 78.628999) (width 0.254) (layer F.Cu) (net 4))
 (segment (start 77.104999 88.534999) (end 78.232 89.662) (width 0.254) (layer B.Cu) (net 4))
 (segment (start 77.104999 78.343001) (end 77.104999 88.534999) (width 0.254) (layer B.Cu) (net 4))
 (segment (start 78.232 77.216) (end 77.104999 78.343001) (width 0.254) (layer B.Cu) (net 4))
 (segment (start 93.472 96.229) (end 93.472 89.662) (width 0.254) (layer B.Cu) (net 4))
 (segment (start 94.073 96.83) (end 93.472 96.229) (width 0.254) (layer B.Cu) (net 4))
 (segment (start 94.8105 96.83) (end 94.073 96.83) (width 0.254) (layer B.Cu) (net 4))
 (segment (start 90.932 72.263) (end 90.932 77.216) (width 0.254) (layer F.Cu) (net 4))
 (segment (start 78.232 87.376) (end 78.232 82.042) (width 0.254) (layer B.Cu) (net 13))
 (segment (start 80.772 82.042) (end 80.772 87.376) (width 0.254) (layer B.Cu) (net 12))
 (segment (start 101.092 87.376) (end 101.092 88.773) (width 0.254) (layer B.Cu) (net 14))
 (segment (start 100.203 89.662) (end 98.552 89.662) (width 0.254) (layer B.Cu) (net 14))
 (segment (start 101.092 88.773) (end 100.203 89.662) (width 0.254) (layer B.Cu) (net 14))
 (segment (start 98.552 87.376) (end 98.552 82.042) (width 0.254) (layer B.Cu) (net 3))
 (segment (start 96.012 82.042) (end 96.012 87.376) (width 0.254) (layer B.Cu) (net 5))
 (segment (start 93.472 87.376) (end 93.472 82.042) (width 0.254) (layer B.Cu) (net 6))
 (segment (start 90.932 87.376) (end 90.932 82.042) (width 0.254) (layer B.Cu) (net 8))
 (segment (start 88.392 87.376) (end 88.392 82.042) (width 0.254) (layer B.Cu) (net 9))
 (segment (start 85.852 87.376) (end 85.852 82.042) (width 0.254) (layer B.Cu) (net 10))
 (segment (start 83.312 87.376) (end 83.312 82.042) (width 0.254) (layer B.Cu) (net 11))
 (segment (start 79.872 94.932) (end 79.915 94.889) (width 0.254) (layer B.Cu) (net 23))
 (segment (start 77.597 94.932) (end 79.872 94.932) (width 0.254) (layer B.Cu) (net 23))
 (segment (start 82.856 98.155) (end 82.026 98.155) (width 0.254) (layer B.Cu) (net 23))
 (segment (start 82.026 98.155) (end 81.534 97.663) (width 0.254) (layer B.Cu) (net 23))
 (segment (start 81.534 97.663) (end 81.534 95.377) (width 0.254) (layer B.Cu) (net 23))
 (segment (start 81.534 95.377) (end 81.026 94.869) (width 0.254) (layer B.Cu) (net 23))
 (segment (start 79.935 94.869) (end 79.915 94.889) (width 0.254) (layer B.Cu) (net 23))
 (segment (start 81.026 94.869) (end 79.935 94.869) (width 0.254) (layer B.Cu) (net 23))
 (segment (start 83.005 92.964) (end 79.883 92.964) (width 0.254) (layer B.Cu) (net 20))
 (segment (start 79.312 91.948) (end 79.312 92.647) (width 0.254) (layer B.Cu) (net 20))
 (segment (start 79.629 92.964) (end 79.883 92.964) (width 0.254) (layer B.Cu) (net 20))
 (segment (start 79.312 92.647) (end 79.629 92.964) (width 0.254) (layer B.Cu) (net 20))
 (segment (start 80.962 91.948) (end 81.788 91.948) (width 0.254) (layer B.Cu) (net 7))
 (segment (start 82.1055 90.8685) (end 82.1055 91.6305) (width 0.254) (layer B.Cu) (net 7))
 (segment (start 83.312 89.662) (end 82.1055 90.8685) (width 0.254) (layer B.Cu) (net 7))
 (segment (start 81.788 91.948) (end 82.1055 91.6305) (width 0.254) (layer B.Cu) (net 7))
 (segment (start 83.312 89.662) (end 85.852 89.662) (width 0.254) (layer B.Cu) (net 7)))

